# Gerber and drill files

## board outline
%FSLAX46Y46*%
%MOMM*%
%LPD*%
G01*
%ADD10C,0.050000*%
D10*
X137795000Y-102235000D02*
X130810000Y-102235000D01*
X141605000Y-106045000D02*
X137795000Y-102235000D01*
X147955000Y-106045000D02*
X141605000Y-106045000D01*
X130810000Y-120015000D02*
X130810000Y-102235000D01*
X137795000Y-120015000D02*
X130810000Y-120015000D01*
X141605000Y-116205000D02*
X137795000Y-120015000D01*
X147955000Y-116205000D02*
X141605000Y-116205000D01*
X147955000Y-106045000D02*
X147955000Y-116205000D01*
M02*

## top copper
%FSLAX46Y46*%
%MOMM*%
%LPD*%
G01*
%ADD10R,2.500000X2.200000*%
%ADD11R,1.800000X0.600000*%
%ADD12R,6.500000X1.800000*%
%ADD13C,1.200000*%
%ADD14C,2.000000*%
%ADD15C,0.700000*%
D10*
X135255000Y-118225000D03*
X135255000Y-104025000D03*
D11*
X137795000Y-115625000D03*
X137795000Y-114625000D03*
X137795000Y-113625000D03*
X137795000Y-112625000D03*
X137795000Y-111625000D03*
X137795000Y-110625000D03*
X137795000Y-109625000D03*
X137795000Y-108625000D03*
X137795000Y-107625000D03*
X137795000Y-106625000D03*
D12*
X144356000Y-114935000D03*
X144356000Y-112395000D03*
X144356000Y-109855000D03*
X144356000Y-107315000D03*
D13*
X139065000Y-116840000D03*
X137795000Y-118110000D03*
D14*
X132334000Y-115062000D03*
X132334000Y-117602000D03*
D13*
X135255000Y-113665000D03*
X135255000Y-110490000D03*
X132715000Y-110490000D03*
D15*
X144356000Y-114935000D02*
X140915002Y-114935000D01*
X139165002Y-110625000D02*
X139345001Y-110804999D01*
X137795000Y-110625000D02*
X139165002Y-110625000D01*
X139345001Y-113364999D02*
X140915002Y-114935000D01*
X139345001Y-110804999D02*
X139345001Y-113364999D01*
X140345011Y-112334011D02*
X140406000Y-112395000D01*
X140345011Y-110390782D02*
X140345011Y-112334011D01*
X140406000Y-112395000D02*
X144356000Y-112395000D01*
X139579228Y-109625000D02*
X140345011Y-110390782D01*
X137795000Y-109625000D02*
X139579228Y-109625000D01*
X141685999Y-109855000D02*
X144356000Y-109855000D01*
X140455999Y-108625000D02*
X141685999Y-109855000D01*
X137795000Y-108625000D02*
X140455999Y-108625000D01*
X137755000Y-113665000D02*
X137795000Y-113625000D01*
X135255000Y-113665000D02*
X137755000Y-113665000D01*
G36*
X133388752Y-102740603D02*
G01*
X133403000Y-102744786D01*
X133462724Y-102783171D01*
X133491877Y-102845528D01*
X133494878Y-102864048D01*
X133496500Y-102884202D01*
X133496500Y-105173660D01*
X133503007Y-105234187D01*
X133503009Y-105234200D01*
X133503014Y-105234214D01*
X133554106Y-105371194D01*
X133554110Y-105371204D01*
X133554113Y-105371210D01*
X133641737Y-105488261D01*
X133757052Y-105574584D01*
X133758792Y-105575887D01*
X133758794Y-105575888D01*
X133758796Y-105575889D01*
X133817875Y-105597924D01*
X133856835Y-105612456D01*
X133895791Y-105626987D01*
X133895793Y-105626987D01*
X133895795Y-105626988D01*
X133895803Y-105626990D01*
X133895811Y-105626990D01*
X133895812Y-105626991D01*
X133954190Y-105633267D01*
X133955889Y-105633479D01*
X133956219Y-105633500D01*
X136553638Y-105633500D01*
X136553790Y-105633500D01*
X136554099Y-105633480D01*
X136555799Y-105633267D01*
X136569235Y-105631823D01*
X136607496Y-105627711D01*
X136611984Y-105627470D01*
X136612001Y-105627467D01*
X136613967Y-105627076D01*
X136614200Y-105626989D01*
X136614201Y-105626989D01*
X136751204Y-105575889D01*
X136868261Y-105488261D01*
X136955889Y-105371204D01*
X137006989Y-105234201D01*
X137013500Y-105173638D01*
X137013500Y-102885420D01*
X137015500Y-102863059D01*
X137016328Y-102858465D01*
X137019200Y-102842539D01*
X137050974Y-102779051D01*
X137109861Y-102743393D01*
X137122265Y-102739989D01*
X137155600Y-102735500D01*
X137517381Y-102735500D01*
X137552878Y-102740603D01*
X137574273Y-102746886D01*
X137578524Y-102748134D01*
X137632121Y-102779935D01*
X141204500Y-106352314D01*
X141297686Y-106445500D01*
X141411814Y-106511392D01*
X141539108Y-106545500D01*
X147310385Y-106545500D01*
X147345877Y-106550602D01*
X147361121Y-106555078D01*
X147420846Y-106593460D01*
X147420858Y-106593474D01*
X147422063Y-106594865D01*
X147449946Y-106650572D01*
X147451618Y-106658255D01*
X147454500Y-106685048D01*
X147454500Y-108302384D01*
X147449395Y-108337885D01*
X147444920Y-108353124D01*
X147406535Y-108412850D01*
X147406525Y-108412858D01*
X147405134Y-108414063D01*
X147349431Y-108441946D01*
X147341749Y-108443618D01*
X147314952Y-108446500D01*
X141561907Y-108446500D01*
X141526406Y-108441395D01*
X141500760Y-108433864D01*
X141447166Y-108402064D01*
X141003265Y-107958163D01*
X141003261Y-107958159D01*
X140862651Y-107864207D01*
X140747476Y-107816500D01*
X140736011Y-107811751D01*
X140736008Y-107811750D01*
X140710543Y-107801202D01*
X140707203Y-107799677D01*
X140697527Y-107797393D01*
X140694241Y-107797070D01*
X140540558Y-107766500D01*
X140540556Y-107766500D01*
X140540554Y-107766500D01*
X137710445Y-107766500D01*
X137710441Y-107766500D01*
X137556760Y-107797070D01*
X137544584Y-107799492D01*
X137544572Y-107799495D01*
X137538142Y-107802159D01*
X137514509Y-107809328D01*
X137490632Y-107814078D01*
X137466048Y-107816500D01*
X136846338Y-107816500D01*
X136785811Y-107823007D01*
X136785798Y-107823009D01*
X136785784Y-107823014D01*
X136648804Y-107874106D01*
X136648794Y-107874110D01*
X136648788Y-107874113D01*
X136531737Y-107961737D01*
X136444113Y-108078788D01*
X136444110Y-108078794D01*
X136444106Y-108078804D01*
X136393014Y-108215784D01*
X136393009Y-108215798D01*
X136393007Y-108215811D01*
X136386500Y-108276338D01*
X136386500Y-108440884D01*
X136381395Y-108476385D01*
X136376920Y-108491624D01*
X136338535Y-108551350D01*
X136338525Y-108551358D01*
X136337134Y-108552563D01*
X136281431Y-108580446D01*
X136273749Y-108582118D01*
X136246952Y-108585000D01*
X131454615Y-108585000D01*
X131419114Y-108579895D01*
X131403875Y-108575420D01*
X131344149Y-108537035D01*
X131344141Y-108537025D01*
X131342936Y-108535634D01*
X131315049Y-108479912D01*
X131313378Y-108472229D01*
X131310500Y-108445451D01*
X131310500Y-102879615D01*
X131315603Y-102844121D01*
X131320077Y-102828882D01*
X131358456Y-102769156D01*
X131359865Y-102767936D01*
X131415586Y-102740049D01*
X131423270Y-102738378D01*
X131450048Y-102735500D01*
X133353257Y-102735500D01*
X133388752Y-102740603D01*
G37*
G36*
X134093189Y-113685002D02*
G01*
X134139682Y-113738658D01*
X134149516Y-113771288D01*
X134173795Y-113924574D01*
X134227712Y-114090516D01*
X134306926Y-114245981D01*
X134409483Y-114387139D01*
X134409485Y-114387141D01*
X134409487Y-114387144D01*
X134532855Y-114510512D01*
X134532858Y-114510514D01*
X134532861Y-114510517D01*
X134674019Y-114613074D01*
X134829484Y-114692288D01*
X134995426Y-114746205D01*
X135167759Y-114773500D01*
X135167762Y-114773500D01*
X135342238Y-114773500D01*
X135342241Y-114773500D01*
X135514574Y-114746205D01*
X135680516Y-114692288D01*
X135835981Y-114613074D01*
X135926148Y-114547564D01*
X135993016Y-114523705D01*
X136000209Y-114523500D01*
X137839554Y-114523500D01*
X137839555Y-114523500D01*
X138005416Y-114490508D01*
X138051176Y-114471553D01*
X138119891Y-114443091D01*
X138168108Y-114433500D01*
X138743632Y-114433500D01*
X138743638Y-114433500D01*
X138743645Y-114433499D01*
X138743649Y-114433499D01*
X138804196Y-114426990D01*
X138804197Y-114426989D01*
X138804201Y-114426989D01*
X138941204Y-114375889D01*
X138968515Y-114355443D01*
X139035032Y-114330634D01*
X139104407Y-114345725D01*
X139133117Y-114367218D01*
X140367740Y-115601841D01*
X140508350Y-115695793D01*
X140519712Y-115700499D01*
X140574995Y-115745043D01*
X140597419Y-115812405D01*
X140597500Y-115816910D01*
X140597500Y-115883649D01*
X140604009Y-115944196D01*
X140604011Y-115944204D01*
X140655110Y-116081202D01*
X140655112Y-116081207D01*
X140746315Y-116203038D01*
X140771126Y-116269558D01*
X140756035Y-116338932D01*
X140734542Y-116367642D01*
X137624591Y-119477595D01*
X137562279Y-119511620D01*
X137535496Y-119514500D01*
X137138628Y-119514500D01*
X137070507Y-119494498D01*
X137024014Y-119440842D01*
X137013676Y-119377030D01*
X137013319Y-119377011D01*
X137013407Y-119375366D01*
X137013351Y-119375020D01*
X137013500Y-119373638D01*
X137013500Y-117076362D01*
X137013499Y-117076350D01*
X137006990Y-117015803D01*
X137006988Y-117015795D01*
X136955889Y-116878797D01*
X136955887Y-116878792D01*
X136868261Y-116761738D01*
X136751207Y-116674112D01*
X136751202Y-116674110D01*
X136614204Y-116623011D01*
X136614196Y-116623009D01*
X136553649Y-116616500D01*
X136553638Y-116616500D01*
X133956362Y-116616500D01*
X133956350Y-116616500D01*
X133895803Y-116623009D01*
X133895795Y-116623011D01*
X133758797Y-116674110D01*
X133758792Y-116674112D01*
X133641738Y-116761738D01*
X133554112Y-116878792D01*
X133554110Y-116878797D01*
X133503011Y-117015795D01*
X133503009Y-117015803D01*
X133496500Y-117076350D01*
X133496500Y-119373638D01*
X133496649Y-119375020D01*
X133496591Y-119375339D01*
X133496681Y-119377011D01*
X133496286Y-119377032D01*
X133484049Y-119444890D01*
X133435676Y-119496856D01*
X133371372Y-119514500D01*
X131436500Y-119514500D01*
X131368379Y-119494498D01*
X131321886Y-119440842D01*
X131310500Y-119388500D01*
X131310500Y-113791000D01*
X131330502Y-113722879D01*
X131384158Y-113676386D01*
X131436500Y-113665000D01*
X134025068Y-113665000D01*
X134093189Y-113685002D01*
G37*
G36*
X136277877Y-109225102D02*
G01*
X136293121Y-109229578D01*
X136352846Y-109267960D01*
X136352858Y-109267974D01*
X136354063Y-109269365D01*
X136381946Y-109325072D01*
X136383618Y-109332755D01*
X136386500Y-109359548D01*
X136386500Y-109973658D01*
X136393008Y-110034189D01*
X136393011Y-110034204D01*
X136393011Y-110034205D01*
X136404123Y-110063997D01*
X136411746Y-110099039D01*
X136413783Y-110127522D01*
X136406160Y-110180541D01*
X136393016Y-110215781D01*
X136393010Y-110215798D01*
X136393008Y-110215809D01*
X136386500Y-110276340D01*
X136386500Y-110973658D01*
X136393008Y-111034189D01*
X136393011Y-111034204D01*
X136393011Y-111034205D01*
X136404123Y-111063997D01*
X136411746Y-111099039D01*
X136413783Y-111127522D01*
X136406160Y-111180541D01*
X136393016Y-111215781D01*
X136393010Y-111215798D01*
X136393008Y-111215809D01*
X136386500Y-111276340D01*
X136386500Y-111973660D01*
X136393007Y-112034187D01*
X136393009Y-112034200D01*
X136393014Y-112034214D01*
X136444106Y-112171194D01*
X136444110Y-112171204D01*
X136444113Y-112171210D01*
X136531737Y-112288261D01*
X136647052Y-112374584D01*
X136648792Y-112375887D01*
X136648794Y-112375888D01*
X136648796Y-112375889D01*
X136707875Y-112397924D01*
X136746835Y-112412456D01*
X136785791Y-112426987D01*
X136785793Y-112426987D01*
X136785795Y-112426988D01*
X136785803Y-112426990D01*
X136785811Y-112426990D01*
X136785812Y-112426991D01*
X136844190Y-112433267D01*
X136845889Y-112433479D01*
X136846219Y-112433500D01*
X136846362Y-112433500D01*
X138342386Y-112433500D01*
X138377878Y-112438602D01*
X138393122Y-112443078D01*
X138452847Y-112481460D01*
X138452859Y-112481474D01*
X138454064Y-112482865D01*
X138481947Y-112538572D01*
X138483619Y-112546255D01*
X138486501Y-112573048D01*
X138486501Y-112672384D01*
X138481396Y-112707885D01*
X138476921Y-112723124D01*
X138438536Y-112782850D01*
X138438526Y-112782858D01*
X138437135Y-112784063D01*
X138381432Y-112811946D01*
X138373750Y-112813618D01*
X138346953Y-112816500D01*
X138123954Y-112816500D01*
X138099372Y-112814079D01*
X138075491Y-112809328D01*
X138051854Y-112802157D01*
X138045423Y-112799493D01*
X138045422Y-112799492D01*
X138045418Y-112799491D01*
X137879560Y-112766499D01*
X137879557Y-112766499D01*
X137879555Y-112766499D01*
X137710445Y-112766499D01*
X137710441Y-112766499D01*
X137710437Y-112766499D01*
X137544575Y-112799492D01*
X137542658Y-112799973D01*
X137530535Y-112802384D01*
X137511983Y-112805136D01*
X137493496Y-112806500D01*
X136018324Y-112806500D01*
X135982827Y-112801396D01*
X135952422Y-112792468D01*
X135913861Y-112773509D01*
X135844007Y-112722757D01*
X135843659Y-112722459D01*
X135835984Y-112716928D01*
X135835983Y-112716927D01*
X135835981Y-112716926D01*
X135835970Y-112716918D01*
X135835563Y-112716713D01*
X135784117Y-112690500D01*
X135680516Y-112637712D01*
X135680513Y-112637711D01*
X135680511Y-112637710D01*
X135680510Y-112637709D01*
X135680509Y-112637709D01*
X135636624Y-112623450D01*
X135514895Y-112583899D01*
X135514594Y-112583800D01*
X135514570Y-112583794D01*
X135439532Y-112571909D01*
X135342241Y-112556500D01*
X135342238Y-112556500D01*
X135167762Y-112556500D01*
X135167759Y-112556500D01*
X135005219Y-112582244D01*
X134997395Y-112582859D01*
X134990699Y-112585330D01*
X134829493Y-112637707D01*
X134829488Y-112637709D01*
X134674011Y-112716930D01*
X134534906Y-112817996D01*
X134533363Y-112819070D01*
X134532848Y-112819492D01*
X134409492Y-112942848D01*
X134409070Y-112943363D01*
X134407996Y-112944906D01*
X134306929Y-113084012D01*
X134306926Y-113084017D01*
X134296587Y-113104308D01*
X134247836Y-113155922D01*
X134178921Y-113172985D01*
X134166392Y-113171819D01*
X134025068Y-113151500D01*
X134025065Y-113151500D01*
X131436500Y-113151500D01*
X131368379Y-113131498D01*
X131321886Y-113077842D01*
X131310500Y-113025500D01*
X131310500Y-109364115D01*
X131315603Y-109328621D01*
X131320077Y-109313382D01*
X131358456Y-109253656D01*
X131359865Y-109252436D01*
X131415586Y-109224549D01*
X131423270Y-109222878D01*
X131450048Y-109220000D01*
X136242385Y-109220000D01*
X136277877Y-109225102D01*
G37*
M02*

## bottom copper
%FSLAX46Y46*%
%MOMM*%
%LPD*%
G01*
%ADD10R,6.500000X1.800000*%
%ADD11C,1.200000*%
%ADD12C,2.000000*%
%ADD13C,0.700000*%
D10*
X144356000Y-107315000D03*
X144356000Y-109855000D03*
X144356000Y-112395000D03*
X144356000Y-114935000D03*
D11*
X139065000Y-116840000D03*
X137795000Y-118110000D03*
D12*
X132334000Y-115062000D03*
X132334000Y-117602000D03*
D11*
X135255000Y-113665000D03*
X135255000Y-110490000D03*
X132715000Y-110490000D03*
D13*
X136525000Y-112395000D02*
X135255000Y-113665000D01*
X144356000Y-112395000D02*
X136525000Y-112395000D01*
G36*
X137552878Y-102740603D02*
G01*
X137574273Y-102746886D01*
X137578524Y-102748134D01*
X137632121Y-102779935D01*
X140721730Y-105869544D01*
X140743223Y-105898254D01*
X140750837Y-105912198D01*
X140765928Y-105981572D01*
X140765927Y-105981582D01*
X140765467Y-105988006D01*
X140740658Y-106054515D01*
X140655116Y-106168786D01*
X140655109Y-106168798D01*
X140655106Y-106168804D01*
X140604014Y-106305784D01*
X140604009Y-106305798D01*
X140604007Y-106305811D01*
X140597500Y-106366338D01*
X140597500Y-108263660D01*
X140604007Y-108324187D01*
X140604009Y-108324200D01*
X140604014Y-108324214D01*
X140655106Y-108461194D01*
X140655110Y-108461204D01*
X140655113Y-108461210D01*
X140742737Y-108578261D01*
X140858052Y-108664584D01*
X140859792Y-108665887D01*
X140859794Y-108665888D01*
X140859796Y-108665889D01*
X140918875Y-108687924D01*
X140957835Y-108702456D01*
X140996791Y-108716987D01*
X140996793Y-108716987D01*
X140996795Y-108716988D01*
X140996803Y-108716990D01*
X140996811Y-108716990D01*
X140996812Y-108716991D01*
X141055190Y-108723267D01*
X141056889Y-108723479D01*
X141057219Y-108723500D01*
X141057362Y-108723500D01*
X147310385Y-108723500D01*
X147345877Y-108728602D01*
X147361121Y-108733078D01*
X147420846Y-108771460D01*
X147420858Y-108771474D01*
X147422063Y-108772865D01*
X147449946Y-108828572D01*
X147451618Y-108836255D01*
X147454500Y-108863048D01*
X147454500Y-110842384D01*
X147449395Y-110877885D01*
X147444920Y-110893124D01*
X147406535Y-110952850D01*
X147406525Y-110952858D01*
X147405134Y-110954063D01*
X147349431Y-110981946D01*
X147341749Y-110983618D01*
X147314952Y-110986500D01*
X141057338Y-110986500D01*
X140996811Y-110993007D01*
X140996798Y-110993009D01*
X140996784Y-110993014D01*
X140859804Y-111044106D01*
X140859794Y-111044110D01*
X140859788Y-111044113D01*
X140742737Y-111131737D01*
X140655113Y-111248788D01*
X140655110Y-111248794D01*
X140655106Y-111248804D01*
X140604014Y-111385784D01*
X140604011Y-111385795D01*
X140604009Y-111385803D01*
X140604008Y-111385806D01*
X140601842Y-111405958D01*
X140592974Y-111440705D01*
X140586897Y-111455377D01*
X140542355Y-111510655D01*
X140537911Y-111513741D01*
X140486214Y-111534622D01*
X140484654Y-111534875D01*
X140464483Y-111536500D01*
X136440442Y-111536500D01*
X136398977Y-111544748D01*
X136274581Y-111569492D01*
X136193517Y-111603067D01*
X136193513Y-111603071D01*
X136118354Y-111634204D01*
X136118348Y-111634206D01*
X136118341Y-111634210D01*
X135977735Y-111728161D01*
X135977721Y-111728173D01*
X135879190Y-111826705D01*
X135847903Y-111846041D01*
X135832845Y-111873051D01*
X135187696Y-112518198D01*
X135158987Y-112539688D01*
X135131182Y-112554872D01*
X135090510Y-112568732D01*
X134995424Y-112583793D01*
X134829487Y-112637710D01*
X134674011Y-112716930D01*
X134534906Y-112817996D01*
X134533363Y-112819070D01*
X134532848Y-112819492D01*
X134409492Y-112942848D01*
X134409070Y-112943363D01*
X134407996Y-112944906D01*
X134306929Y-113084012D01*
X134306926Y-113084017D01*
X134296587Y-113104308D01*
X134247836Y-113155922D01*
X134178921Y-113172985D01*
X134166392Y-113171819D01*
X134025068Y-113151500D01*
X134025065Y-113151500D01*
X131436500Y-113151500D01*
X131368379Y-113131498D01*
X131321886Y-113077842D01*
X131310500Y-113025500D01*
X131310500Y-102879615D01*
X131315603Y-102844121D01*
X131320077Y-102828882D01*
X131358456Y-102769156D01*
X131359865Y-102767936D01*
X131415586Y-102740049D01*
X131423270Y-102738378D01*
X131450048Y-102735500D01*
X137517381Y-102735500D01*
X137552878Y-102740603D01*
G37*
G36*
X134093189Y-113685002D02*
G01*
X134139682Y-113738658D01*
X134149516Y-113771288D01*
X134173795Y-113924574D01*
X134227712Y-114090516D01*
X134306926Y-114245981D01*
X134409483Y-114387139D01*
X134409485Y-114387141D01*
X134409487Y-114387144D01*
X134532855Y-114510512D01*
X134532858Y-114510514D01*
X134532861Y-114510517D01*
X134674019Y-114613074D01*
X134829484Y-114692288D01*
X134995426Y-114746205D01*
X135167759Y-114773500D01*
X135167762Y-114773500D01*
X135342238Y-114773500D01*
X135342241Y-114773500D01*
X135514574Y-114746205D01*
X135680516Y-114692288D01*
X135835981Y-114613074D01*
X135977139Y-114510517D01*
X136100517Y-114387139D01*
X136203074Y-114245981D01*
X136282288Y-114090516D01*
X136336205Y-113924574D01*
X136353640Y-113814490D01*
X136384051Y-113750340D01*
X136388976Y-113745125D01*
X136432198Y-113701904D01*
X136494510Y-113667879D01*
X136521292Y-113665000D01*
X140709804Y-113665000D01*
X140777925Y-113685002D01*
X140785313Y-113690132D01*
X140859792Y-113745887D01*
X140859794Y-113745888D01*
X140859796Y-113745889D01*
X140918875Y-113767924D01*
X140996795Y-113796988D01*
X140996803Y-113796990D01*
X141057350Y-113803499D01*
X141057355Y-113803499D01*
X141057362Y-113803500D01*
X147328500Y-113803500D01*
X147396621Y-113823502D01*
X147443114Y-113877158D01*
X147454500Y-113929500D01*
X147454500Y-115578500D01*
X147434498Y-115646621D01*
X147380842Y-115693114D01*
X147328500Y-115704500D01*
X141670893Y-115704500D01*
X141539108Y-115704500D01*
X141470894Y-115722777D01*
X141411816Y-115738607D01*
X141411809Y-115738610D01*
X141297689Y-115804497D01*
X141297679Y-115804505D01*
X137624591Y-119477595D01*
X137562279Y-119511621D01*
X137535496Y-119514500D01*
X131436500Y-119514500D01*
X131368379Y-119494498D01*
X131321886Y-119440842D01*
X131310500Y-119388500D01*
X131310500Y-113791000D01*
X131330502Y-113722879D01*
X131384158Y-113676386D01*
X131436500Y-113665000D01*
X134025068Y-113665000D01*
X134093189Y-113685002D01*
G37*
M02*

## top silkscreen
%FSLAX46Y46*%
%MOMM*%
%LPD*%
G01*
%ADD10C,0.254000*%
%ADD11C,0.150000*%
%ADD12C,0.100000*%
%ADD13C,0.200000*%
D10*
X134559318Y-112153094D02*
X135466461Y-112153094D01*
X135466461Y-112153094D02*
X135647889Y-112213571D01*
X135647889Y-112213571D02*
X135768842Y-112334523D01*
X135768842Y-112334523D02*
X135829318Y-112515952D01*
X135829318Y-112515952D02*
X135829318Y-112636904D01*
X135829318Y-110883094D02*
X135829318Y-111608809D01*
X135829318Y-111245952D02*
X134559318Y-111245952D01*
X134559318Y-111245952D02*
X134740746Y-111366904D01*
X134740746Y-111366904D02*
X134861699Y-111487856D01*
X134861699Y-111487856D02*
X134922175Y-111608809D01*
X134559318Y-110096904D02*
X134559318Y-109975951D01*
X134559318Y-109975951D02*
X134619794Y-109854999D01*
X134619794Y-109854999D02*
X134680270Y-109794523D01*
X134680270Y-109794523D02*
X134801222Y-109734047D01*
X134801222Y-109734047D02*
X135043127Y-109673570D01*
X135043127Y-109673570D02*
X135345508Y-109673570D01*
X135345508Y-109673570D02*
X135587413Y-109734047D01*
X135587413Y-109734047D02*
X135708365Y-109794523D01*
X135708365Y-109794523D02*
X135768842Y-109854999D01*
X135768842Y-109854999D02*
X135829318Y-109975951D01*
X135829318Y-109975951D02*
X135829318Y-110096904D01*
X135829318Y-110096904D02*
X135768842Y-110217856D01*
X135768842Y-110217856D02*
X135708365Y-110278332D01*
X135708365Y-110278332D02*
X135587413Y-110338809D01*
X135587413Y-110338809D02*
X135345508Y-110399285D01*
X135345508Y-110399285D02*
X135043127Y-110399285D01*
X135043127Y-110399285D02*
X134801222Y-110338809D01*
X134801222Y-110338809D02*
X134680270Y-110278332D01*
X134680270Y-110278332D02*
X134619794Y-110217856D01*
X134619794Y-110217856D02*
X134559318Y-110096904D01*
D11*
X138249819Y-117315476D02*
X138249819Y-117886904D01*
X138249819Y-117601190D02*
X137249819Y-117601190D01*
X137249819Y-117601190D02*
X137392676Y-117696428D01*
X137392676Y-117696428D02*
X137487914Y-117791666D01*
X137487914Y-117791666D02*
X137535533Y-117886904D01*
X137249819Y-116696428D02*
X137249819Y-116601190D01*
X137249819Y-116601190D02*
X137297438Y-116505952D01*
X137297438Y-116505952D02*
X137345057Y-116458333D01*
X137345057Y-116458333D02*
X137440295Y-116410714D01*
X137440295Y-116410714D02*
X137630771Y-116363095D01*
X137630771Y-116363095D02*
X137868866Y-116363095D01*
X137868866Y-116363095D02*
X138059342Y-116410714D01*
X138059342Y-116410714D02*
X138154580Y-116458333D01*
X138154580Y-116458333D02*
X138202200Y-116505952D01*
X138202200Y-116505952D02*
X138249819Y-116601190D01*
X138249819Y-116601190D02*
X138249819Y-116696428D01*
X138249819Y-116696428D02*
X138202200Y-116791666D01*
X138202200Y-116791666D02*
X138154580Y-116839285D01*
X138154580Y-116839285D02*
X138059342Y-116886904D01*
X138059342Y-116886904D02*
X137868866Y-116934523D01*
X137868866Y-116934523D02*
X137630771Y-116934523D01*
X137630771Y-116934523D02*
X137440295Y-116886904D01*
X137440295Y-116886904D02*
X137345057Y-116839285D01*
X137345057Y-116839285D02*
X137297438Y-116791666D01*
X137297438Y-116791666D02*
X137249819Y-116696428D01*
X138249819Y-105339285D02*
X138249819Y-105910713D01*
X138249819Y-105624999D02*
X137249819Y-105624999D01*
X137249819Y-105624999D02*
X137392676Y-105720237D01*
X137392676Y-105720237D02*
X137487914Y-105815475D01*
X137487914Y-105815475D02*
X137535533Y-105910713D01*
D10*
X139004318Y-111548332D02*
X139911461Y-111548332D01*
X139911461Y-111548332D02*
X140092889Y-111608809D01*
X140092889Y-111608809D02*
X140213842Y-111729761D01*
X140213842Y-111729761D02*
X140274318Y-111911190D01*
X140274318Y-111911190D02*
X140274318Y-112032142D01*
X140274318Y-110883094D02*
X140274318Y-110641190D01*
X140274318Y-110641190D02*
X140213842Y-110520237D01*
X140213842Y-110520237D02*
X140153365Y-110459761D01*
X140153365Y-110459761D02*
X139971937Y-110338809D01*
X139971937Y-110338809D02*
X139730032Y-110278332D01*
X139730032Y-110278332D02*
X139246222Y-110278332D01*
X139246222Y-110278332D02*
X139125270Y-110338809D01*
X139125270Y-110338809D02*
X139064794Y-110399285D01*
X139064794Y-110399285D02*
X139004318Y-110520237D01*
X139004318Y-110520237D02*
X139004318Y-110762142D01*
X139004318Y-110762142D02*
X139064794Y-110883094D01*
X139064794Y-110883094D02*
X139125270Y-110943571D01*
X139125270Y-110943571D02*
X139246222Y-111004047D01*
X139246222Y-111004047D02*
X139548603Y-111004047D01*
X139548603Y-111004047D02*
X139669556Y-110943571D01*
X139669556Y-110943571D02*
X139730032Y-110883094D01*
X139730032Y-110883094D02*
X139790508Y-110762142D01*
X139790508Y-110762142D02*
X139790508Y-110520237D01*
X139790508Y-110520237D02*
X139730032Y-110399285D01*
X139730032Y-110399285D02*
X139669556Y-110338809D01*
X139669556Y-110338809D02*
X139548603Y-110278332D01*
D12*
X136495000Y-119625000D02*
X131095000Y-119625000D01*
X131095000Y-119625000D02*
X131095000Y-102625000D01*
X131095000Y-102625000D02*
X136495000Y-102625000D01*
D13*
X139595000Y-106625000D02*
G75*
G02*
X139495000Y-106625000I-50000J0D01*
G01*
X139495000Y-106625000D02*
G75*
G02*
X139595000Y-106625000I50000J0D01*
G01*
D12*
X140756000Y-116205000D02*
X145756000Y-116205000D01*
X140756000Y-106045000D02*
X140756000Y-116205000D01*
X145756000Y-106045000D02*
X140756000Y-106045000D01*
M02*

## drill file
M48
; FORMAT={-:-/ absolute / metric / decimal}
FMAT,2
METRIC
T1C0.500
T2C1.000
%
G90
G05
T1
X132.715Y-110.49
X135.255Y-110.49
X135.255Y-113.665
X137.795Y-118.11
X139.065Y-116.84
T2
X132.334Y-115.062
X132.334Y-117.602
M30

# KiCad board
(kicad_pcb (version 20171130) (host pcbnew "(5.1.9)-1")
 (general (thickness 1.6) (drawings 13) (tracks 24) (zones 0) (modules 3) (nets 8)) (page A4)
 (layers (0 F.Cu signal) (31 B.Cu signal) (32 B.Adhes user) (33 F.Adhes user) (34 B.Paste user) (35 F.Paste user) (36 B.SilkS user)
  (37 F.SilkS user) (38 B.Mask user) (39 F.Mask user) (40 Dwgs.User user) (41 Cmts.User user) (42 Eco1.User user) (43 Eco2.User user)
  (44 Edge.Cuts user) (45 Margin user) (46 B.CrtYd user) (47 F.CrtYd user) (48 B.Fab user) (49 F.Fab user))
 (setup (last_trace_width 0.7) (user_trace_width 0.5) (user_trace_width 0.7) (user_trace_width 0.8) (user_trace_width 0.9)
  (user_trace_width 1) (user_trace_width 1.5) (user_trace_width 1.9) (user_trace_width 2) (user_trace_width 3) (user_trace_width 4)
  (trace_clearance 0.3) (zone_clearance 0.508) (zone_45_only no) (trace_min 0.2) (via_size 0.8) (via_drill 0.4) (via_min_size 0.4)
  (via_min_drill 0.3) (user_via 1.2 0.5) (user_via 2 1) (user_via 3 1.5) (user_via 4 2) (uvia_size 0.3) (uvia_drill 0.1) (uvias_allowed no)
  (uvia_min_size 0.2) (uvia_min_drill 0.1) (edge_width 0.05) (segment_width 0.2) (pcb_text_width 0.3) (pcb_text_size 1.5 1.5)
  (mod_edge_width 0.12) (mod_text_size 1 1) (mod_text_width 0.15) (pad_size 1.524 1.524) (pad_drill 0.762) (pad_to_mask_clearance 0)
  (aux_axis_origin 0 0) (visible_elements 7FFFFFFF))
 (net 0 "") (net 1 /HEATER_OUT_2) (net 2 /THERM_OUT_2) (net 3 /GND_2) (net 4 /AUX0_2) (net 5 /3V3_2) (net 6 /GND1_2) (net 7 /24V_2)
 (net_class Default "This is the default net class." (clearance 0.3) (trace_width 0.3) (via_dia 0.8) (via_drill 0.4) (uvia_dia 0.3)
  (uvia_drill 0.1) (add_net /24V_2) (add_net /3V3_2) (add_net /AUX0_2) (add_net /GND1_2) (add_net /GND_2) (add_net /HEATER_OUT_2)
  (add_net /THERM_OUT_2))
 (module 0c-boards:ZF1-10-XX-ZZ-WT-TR (layer F.Cu) (at 137.795 111.125 270)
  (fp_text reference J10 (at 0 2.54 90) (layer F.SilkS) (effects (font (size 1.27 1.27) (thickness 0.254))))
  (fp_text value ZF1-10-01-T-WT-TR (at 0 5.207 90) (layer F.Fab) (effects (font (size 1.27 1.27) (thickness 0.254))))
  (fp_line (start 8.5 1.3) (end 8.5 6.7) (layer F.SilkS) (width 0.1))
  (fp_line (start 8.5 6.7) (end -8.5 6.7) (layer F.SilkS) (width 0.1))
  (fp_line (start -8.5 6.7) (end -8.5 1.3) (layer F.SilkS) (width 0.1))
  (fp_circle (center -4.5 -1.75) (end -4.5 -1.7) (layer F.SilkS) (width 0.2))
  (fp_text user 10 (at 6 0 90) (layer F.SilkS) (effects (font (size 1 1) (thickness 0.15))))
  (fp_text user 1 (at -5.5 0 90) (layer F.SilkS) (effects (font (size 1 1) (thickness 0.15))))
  (pad 12 smd rect (at 7.1 2.54 270) (size 2.2 2.5) (layers F.Cu F.Paste F.Mask))
  (pad 11 smd rect (at -7.1 2.54 270) (size 2.2 2.5) (layers F.Cu F.Paste F.Mask))
  (pad 10 smd rect (at 4.5 0 270) (size 0.6 1.8) (layers F.Cu F.Paste F.Mask) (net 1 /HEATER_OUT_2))
  (pad 9 smd rect (at 3.5 0 270) (size 0.6 1.8) (layers F.Cu F.Paste F.Mask) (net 1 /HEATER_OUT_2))
  (pad 8 smd rect (at 2.5 0 270) (size 0.6 1.8) (layers F.Cu F.Paste F.Mask) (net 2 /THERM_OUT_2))
  (pad 7 smd rect (at 1.5 0 270) (size 0.6 1.8) (layers F.Cu F.Paste F.Mask) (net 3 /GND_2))
  (pad 6 smd rect (at 0.5 0 270) (size 0.6 1.8) (layers F.Cu F.Paste F.Mask))
  (pad 5 smd rect (at -0.5 0 270) (size 0.6 1.8) (layers F.Cu F.Paste F.Mask) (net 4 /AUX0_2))
  (pad 4 smd rect (at -1.5 0 270) (size 0.6 1.8) (layers F.Cu F.Paste F.Mask) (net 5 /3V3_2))
  (pad 3 smd rect (at -2.5 0 270) (size 0.6 1.8) (layers F.Cu F.Paste F.Mask) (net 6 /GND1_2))
  (pad 2 smd rect (at -3.5 0 270) (size 0.6 1.8) (layers F.Cu F.Paste F.Mask) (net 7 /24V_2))
  (pad 1 smd rect (at -4.5 0 270) (size 0.6 1.8) (layers F.Cu F.Paste F.Mask) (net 7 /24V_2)))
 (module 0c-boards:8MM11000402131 (layer F.Cu) (at 144.145 111.125 270)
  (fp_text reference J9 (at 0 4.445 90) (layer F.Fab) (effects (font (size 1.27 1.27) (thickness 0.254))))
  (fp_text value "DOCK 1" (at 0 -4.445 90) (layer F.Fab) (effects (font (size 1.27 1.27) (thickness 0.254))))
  (fp_line (start 5.08 3.389) (end 5.08 -1.611) (layer F.SilkS) (width 0.1))
  (fp_line (start -5.08 3.389) (end 5.08 3.389) (layer F.SilkS) (width 0.1))
  (fp_line (start -5.08 -1.611) (end -5.08 3.389) (layer F.SilkS) (width 0.1))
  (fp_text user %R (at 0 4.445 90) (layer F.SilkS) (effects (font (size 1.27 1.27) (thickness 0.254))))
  (pad 4 smd rect (at 3.81 -0.211 270) (size 1.8 6.5) (layers F.Cu F.Paste F.Mask) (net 4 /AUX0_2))
  (pad 3 smd rect (at 1.27 -0.211 270) (size 1.8 6.5) (layers F.Cu F.Paste F.Mask) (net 5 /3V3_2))
  (pad 2 smd rect (at -1.27 -0.211 270) (size 1.8 6.5) (layers F.Cu F.Paste F.Mask) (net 6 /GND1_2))
  (pad 1 smd rect (at -3.81 -0.211 270) (size 1.8 6.5) (layers F.Cu F.Paste F.Mask) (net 7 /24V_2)))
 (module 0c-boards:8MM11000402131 (layer B.Cu) (at 144.145 111.125 90)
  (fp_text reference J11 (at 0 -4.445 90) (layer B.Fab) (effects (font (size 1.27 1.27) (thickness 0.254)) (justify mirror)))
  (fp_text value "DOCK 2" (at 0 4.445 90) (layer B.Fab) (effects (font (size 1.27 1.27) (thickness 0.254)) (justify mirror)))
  (pad 4 smd rect (at 3.81 0.211 90) (size 1.8 6.5) (layers B.Cu B.Paste B.Mask))
  (pad 3 smd rect (at 1.27 0.211 90) (size 1.8 6.5) (layers B.Cu B.Paste B.Mask) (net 3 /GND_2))
  (pad 2 smd rect (at -1.27 0.211 90) (size 1.8 6.5) (layers B.Cu B.Paste B.Mask) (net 2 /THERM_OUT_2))
  (pad 1 smd rect (at -3.81 0.211 90) (size 1.8 6.5) (layers B.Cu B.Paste B.Mask) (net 1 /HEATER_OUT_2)))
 (gr_line (start 137.795 102.235) (end 130.81 102.235) (layer Edge.Cuts) (width 0.05))
 (gr_line (start 141.605 106.045) (end 137.795 102.235) (layer Edge.Cuts) (width 0.05))
 (gr_line (start 147.955 106.045) (end 141.605 106.045) (layer Edge.Cuts) (width 0.05))
 (gr_line (start 130.81 120.015) (end 130.81 102.235) (layer Edge.Cuts) (width 0.05))
 (gr_line (start 137.795 120.015) (end 130.81 120.015) (layer Edge.Cuts) (width 0.05))
 (gr_line (start 141.605 116.205) (end 137.795 120.015) (layer Edge.Cuts) (width 0.05))
 (gr_line (start 147.955 116.205) (end 141.605 116.205) (layer Edge.Cuts) (width 0.05))
 (gr_line (start 147.955 106.045) (end 147.955 116.205) (layer Edge.Cuts) (width 0.05))
 (segment (start 144.356 114.935) (end 140.915002 114.935) (width 0.7) (layer F.Cu) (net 4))
 (segment (start 139.165002 110.625) (end 139.345001 110.804999) (width 0.7) (layer F.Cu) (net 4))
 (segment (start 137.795 110.625) (end 139.165002 110.625) (width 0.7) (layer F.Cu) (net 4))
 (segment (start 139.345001 113.364999) (end 140.915002 114.935) (width 0.7) (layer F.Cu) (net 4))
 (segment (start 139.345001 110.804999) (end 139.345001 113.364999) (width 0.7) (layer F.Cu) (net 4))
 (segment (start 140.345011 112.334011) (end 140.406 112.395) (width 0.7) (layer F.Cu) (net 5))
 (segment (start 140.345011 110.390782) (end 140.345011 112.334011) (width 0.7) (layer F.Cu) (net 5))
 (segment (start 140.406 112.395) (end 144.356 112.395) (width 0.7) (layer F.Cu) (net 5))
 (segment (start 139.579228 109.625) (end 140.345011 110.390782) (width 0.7) (layer F.Cu) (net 5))
 (segment (start 137.795 109.625) (end 139.579228 109.625) (width 0.7) (layer F.Cu) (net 5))
 (segment (start 141.685999 109.855) (end 144.356 109.855) (width 0.7) (layer F.Cu) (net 6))
 (segment (start 140.455999 108.625) (end 141.685999 109.855) (width 0.7) (layer F.Cu) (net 6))
 (segment (start 137.795 108.625) (end 140.455999 108.625) (width 0.7) (layer F.Cu) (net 6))
 (via (at 139.065 116.84) (size 1.2) (drill 0.5) (layers F.Cu B.Cu) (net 1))
 (via (at 137.795 118.11) (size 1.2) (drill 0.5) (layers F.Cu B.Cu) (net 1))
 (via (at 132.334 115.062) (size 2) (drill 1) (layers F.Cu B.Cu) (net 1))
 (via (at 132.334 117.602) (size 2) (drill 1) (layers F.Cu B.Cu) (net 1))
 (via (at 135.255 113.665) (size 1.2) (drill 0.5) (layers F.Cu B.Cu) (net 2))
 (segment (start 136.525 112.395) (end 135.255 113.665) (width 0.7) (layer B.Cu) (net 2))
 (segment (start 144.356 112.395) (end 136.525 112.395) (width 0.7) (layer B.Cu) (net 2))
 (segment (start 137.755 113.665) (end 137.795 113.625) (width 0.7) (layer F.Cu) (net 2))
 (segment (start 135.255 113.665) (end 137.755 113.665) (width 0.7) (layer F.Cu) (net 2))
 (via (at 135.255 110.49) (size 1.2) (drill 0.5) (layers F.Cu B.Cu) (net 3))
 (via (at 132.715 110.49) (size 1.2) (drill 0.5) (layers F.Cu B.Cu) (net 3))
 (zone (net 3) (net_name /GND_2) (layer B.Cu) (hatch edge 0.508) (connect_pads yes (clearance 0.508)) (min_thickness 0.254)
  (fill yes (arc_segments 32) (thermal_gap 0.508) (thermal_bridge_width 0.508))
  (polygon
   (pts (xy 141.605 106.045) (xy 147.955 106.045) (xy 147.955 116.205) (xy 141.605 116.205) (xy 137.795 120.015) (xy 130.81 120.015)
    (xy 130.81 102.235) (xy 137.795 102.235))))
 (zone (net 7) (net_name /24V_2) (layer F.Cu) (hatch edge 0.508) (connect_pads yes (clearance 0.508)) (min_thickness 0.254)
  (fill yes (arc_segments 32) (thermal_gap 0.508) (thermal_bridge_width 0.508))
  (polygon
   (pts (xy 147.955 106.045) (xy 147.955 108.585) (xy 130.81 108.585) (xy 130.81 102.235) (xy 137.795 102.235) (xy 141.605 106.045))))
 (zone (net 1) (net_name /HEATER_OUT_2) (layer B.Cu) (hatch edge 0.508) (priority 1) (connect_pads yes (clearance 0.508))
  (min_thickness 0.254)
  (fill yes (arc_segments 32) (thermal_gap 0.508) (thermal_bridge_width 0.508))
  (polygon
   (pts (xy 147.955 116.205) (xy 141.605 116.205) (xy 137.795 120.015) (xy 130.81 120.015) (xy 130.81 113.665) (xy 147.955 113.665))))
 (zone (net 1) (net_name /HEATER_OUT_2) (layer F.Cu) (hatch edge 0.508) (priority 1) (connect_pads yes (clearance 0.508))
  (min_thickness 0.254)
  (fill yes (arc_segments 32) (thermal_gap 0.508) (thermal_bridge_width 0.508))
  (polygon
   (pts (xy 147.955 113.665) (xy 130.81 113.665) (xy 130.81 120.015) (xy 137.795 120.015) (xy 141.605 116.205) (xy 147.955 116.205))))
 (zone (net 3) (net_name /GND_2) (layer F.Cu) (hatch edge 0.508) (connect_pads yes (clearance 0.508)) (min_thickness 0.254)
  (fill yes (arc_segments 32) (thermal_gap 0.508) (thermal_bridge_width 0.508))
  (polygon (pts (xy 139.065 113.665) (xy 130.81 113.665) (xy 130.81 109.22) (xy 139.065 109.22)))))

